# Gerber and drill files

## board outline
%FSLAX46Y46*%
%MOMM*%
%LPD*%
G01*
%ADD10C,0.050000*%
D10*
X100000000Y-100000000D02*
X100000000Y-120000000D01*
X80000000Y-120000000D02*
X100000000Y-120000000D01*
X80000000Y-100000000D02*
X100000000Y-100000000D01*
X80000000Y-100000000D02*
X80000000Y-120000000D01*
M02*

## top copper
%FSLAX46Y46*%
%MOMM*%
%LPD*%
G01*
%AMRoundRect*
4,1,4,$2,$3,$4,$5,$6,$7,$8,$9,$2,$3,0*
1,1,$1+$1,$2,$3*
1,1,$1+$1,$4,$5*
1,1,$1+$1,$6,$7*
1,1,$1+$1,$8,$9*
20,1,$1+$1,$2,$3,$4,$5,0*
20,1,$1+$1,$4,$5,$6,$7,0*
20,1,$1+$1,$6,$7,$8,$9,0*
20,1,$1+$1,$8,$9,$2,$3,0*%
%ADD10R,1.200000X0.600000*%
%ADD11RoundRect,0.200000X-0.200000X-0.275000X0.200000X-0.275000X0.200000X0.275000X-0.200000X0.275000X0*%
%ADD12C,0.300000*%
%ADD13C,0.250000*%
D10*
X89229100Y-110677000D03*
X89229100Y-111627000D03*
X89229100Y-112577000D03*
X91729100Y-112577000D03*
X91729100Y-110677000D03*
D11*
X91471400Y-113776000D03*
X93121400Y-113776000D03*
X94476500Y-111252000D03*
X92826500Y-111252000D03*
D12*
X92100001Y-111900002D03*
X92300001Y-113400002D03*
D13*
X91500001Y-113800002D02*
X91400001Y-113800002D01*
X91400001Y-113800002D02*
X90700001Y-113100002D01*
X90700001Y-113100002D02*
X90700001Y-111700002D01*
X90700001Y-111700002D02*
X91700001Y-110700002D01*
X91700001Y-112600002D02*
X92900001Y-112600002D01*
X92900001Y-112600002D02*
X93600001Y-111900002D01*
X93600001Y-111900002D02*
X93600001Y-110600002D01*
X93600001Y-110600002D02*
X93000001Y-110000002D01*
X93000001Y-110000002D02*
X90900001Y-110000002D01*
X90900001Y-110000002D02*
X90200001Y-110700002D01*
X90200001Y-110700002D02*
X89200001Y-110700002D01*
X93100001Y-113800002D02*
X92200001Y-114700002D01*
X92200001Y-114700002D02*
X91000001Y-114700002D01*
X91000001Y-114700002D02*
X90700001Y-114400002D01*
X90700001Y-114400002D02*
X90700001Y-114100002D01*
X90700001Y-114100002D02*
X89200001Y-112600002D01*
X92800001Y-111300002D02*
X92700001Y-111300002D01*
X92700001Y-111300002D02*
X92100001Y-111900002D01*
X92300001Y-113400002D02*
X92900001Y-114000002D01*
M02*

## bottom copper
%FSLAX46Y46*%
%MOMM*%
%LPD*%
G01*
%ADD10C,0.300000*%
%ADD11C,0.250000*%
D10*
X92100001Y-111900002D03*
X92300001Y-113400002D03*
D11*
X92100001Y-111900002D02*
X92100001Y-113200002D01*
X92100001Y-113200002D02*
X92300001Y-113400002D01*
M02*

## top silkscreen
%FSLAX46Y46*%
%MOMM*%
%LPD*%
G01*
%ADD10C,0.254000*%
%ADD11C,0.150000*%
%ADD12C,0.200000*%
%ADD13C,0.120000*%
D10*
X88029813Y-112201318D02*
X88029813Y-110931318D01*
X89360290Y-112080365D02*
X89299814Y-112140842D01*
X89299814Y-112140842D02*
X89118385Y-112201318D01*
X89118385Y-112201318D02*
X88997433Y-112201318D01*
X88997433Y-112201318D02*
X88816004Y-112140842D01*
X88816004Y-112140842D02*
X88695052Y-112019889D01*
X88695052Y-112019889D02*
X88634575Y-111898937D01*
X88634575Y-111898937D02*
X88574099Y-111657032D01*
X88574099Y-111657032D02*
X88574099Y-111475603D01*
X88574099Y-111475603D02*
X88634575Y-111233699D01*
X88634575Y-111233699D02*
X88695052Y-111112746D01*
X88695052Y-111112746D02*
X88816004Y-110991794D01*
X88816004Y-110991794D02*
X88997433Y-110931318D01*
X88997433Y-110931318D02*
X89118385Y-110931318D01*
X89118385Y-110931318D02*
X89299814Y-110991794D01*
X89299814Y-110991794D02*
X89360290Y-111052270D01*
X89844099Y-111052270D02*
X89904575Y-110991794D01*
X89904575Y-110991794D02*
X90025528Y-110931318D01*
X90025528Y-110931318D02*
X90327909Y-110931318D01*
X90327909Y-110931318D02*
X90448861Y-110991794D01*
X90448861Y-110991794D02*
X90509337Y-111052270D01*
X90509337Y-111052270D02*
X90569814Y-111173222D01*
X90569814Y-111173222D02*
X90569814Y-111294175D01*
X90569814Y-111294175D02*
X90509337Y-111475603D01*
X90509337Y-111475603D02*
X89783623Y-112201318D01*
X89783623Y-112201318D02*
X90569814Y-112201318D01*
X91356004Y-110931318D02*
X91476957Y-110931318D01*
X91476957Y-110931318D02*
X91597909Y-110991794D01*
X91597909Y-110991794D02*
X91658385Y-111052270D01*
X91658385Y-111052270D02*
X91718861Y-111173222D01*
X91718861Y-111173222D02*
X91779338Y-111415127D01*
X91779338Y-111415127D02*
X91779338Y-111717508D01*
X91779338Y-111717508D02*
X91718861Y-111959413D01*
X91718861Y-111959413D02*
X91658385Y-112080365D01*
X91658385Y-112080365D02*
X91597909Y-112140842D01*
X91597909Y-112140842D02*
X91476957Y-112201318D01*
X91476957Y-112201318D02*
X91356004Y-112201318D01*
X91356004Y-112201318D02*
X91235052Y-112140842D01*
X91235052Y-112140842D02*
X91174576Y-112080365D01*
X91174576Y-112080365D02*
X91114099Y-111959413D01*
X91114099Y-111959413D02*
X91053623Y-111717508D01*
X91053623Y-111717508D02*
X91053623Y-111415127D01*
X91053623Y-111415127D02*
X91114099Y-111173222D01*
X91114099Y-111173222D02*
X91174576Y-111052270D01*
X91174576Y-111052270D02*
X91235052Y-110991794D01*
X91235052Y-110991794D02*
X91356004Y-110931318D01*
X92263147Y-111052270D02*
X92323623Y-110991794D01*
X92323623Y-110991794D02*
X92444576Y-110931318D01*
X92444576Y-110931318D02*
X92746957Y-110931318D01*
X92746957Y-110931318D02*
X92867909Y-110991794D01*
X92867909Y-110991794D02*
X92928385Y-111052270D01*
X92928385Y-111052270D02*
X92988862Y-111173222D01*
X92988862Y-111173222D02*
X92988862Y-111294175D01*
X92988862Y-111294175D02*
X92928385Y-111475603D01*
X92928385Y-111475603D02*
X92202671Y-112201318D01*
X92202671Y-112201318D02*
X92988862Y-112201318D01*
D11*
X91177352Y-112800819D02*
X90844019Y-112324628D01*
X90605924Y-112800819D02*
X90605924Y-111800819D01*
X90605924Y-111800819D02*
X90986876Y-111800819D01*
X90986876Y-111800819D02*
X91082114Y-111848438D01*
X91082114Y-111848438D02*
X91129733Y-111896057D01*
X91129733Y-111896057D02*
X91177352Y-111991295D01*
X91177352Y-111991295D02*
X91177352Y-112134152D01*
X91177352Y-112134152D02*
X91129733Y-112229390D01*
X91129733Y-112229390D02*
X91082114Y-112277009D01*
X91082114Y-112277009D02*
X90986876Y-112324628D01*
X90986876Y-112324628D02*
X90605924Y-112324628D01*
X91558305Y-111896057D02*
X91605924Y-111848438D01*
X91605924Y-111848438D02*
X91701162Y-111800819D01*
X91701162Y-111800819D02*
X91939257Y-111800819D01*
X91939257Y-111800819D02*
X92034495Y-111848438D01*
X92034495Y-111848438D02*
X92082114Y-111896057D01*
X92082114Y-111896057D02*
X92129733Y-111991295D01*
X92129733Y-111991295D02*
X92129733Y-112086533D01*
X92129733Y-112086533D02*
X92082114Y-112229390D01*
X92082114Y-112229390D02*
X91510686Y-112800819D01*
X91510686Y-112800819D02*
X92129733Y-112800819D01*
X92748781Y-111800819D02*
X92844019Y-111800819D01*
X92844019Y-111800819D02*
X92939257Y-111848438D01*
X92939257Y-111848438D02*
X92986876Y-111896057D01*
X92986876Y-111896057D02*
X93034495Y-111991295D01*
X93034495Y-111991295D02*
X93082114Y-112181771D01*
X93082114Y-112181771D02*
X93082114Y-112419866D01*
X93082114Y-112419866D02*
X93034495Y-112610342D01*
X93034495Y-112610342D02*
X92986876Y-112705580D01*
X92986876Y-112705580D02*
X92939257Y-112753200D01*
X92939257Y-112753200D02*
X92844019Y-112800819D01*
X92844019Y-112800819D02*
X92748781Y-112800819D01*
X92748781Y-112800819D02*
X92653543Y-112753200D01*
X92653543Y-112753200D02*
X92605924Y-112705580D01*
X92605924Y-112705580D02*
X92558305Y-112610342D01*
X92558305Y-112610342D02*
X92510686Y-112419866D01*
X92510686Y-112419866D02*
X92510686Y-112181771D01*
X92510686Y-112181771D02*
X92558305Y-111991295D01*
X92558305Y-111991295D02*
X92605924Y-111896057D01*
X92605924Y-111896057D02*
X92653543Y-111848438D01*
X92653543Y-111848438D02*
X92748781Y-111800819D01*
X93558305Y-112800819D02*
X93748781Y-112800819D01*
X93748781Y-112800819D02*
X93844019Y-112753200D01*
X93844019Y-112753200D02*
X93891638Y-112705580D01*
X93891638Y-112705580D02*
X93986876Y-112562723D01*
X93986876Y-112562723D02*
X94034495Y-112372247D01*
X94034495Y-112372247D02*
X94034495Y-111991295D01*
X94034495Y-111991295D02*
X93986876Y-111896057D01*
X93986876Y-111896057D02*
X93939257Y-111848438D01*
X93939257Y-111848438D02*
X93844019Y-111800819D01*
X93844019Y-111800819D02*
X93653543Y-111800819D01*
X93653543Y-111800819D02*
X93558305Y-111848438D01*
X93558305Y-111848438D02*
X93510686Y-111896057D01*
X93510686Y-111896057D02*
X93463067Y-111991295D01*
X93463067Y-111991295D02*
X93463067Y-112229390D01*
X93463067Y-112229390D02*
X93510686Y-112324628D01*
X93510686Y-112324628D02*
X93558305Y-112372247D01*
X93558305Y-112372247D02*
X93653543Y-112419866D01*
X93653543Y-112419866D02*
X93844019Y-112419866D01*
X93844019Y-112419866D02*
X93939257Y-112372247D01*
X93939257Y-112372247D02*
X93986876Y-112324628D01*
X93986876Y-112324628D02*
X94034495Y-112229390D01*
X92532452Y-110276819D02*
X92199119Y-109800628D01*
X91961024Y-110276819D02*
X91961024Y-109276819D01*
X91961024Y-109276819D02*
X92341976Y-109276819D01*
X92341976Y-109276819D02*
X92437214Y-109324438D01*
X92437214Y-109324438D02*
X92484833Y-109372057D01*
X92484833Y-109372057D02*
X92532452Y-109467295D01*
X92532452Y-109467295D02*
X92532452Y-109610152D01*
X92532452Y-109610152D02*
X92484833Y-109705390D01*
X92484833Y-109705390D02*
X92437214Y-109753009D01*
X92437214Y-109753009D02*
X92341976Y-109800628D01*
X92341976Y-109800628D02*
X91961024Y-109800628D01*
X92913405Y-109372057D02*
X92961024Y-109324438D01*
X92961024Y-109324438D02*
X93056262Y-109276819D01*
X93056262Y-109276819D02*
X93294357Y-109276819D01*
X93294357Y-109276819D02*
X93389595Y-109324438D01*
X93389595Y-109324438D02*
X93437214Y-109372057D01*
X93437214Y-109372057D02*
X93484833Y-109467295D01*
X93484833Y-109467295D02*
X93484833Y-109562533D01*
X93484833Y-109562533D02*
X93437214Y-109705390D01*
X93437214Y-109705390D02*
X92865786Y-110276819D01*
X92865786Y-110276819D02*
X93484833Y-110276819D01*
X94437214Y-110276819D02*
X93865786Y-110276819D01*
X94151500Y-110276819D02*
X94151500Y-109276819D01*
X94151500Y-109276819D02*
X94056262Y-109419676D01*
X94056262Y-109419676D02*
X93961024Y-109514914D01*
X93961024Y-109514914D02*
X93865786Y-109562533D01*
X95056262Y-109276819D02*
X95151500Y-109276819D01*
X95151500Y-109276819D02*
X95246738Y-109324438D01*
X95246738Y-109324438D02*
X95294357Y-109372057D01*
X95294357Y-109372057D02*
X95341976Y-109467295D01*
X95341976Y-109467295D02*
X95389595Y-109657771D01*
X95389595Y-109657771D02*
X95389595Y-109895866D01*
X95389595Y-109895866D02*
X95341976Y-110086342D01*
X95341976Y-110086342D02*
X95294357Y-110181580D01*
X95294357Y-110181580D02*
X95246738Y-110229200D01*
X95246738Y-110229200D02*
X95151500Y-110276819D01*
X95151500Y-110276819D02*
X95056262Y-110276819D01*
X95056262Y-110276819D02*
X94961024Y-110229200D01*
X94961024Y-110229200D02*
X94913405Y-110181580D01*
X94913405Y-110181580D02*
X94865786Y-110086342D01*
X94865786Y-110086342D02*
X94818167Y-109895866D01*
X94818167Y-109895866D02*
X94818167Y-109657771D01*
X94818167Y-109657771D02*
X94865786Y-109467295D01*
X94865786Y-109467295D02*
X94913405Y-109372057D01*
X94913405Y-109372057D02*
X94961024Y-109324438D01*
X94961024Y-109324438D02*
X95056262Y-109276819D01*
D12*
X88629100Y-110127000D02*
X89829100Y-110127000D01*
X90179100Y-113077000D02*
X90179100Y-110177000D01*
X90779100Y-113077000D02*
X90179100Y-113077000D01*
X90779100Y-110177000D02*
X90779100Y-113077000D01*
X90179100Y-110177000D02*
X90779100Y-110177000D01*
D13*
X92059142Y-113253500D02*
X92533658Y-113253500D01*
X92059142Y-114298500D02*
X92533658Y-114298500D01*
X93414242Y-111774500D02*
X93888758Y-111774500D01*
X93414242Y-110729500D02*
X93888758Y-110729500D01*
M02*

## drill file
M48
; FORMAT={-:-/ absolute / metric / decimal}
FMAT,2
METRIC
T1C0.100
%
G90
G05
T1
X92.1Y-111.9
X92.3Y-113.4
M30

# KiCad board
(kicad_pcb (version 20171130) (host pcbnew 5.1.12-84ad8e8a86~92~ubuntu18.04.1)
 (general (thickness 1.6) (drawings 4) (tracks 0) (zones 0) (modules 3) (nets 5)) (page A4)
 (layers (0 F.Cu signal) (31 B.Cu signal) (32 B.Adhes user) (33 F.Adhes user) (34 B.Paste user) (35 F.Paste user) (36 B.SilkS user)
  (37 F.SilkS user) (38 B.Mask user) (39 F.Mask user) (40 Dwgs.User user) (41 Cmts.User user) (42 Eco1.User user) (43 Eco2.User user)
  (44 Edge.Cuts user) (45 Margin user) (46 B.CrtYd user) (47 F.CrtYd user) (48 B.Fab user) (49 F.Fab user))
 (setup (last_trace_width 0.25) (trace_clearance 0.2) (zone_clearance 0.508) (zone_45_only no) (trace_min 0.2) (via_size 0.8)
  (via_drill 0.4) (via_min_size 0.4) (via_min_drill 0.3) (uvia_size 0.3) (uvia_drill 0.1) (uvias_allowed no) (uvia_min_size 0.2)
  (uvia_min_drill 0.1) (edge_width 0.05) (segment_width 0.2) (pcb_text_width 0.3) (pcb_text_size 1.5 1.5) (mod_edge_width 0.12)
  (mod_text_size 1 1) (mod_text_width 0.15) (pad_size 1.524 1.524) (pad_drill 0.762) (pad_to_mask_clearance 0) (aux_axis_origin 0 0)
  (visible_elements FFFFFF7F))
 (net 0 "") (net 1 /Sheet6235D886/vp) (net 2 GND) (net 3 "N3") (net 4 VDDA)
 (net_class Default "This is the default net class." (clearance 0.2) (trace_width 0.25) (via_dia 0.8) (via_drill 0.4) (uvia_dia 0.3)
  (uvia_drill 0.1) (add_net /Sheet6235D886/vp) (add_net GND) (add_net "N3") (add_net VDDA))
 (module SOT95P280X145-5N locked (layer F.Cu) (at 90.479100 111.627000)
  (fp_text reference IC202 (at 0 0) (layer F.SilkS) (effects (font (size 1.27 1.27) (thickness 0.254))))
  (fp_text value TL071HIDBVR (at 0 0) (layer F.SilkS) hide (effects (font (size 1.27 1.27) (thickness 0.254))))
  (fp_line (start -1.85 -1.5) (end -0.65 -1.5) (layer F.SilkS) (width 0.2))
  (fp_line (start -0.3 1.45) (end -0.3 -1.45) (layer F.SilkS) (width 0.2))
  (fp_line (start 0.3 1.45) (end -0.3 1.45) (layer F.SilkS) (width 0.2))
  (fp_line (start 0.3 -1.45) (end 0.3 1.45) (layer F.SilkS) (width 0.2))
  (fp_line (start -0.3 -1.45) (end 0.3 -1.45) (layer F.SilkS) (width 0.2))
  (pad 1 smd rect (at -1.25 -0.95 90.000000) (size 0.6 1.2) (layers F.Cu F.Mask F.Paste) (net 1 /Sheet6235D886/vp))
  (pad 2 smd rect (at -1.25 0 90.000000) (size 0.6 1.2) (layers F.Cu F.Mask F.Paste) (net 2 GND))
  (pad 3 smd rect (at -1.25 0.95 90.000000) (size 0.6 1.2) (layers F.Cu F.Mask F.Paste) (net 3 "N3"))
  (pad 4 smd rect (at 1.25 0.95 90.000000) (size 0.6 1.2) (layers F.Cu F.Mask F.Paste) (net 1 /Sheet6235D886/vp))
  (pad 5 smd rect (at 1.25 -0.95 90.000000) (size 0.6 1.2) (layers F.Cu F.Mask F.Paste) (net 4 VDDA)))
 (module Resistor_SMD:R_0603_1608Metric (layer F.Cu) (at 92.296400 113.776000)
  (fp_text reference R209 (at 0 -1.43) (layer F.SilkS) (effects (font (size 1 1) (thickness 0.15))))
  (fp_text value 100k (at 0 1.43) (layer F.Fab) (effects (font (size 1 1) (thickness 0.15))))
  (fp_line (start -0.237258 -0.5225) (end 0.237258 -0.5225) (layer F.SilkS) (width 0.12))
  (fp_line (start -0.237258 0.5225) (end 0.237258 0.5225) (layer F.SilkS) (width 0.12))
  (pad 1 smd roundrect (at -0.825 0) (size 0.8 0.95) (layers F.Cu F.Mask F.Paste) (roundrect_rratio 0.25) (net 4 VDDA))
  (pad 2 smd roundrect (at 0.825 0) (size 0.8 0.95) (layers F.Cu F.Mask F.Paste) (roundrect_rratio 0.25) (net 3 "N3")))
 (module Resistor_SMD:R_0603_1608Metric (layer F.Cu) (at 93.651500 111.252000)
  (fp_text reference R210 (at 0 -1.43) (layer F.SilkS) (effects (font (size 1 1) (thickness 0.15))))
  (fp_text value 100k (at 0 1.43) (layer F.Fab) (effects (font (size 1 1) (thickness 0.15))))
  (fp_line (start -0.237258 0.5225) (end 0.237258 0.5225) (layer F.SilkS) (width 0.12))
  (fp_line (start -0.237258 -0.5225) (end 0.237258 -0.5225) (layer F.SilkS) (width 0.12))
  (pad 2 smd roundrect (at 0.825 0) (size 0.8 0.95) (layers F.Cu F.Mask F.Paste) (roundrect_rratio 0.25) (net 2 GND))
  (pad 1 smd roundrect (at -0.825 0) (size 0.8 0.95) (layers F.Cu F.Mask F.Paste) (roundrect_rratio 0.25) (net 3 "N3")))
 (gr_line (start 100 100) (end 100 120) (layer Edge.Cuts) (width 0.05))
 (gr_line (start 80 120) (end 100 120) (layer Edge.Cuts) (width 0.05))
 (gr_line (start 80 100) (end 100 100) (layer Edge.Cuts) (width 0.05))
 (gr_line (start 80 100) (end 80 120) (layer Edge.Cuts) (width 0.05))
 (segment (start 91.500001 113.800002) (end 91.400001 113.800002) (width 0.250000) (layer F.Cu) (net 4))
 (segment (start 91.400001 113.800002) (end 90.700001 113.100002) (width 0.250000) (layer F.Cu) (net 4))
 (segment (start 90.700001 113.100002) (end 90.700001 111.700002) (width 0.250000) (layer F.Cu) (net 4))
 (segment (start 90.700001 111.700002) (end 91.700001 110.700002) (width 0.250000) (layer F.Cu) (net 4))
 (segment (start 91.700001 112.600002) (end 92.900001 112.600002) (width 0.250000) (layer F.Cu) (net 1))
 (segment (start 92.900001 112.600002) (end 93.600001 111.900002) (width 0.250000) (layer F.Cu) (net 1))
 (segment (start 93.600001 111.900002) (end 93.600001 110.600002) (width 0.250000) (layer F.Cu) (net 1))
 (segment (start 93.600001 110.600002) (end 93.000001 110.000002) (width 0.250000) (layer F.Cu) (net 1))
 (segment (start 93.000001 110.000002) (end 90.900001 110.000002) (width 0.250000) (layer F.Cu) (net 1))
 (segment (start 90.900001 110.000002) (end 90.200001 110.700002) (width 0.250000) (layer F.Cu) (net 1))
 (segment (start 90.200001 110.700002) (end 89.200001 110.700002) (width 0.250000) (layer F.Cu) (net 1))
 (segment (start 93.100001 113.800002) (end 92.200001 114.700002) (width 0.250000) (layer F.Cu) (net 3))
 (segment (start 92.200001 114.700002) (end 91.000001 114.700002) (width 0.250000) (layer F.Cu) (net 3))
 (segment (start 91.000001 114.700002) (end 90.700001 114.400002) (width 0.250000) (layer F.Cu) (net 3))
 (segment (start 90.700001 114.400002) (end 90.700001 114.100002) (width 0.250000) (layer F.Cu) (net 3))
 (segment (start 90.700001 114.100002) (end 89.200001 112.600002) (width 0.250000) (layer F.Cu) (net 3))
 (segment (start 92.800001 111.300002) (end 92.700001 111.300002) (width 0.250000) (layer F.Cu) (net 3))
 (segment (start 92.700001 111.300002) (end 92.100001 111.900002) (width 0.250000) (layer F.Cu) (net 3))
 (segment (start 92.100001 111.900002) (end 92.100001 113.200002) (width 0.250000) (layer B.Cu) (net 3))
 (segment (start 92.100001 113.200002) (end 92.300001 113.400002) (width 0.250000) (layer B.Cu) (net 3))
 (segment (start 92.300001 113.400002) (end 92.900001 114.000002) (width 0.250000) (layer F.Cu) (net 3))
 (via micro (at 92.100001 111.900002) (size 0.300000) (drill 0.100000) (layers F.Cu B.Cu) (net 3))
 (via micro (at 92.300001 113.400002) (size 0.300000) (drill 0.100000) (layers F.Cu B.Cu) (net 3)))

